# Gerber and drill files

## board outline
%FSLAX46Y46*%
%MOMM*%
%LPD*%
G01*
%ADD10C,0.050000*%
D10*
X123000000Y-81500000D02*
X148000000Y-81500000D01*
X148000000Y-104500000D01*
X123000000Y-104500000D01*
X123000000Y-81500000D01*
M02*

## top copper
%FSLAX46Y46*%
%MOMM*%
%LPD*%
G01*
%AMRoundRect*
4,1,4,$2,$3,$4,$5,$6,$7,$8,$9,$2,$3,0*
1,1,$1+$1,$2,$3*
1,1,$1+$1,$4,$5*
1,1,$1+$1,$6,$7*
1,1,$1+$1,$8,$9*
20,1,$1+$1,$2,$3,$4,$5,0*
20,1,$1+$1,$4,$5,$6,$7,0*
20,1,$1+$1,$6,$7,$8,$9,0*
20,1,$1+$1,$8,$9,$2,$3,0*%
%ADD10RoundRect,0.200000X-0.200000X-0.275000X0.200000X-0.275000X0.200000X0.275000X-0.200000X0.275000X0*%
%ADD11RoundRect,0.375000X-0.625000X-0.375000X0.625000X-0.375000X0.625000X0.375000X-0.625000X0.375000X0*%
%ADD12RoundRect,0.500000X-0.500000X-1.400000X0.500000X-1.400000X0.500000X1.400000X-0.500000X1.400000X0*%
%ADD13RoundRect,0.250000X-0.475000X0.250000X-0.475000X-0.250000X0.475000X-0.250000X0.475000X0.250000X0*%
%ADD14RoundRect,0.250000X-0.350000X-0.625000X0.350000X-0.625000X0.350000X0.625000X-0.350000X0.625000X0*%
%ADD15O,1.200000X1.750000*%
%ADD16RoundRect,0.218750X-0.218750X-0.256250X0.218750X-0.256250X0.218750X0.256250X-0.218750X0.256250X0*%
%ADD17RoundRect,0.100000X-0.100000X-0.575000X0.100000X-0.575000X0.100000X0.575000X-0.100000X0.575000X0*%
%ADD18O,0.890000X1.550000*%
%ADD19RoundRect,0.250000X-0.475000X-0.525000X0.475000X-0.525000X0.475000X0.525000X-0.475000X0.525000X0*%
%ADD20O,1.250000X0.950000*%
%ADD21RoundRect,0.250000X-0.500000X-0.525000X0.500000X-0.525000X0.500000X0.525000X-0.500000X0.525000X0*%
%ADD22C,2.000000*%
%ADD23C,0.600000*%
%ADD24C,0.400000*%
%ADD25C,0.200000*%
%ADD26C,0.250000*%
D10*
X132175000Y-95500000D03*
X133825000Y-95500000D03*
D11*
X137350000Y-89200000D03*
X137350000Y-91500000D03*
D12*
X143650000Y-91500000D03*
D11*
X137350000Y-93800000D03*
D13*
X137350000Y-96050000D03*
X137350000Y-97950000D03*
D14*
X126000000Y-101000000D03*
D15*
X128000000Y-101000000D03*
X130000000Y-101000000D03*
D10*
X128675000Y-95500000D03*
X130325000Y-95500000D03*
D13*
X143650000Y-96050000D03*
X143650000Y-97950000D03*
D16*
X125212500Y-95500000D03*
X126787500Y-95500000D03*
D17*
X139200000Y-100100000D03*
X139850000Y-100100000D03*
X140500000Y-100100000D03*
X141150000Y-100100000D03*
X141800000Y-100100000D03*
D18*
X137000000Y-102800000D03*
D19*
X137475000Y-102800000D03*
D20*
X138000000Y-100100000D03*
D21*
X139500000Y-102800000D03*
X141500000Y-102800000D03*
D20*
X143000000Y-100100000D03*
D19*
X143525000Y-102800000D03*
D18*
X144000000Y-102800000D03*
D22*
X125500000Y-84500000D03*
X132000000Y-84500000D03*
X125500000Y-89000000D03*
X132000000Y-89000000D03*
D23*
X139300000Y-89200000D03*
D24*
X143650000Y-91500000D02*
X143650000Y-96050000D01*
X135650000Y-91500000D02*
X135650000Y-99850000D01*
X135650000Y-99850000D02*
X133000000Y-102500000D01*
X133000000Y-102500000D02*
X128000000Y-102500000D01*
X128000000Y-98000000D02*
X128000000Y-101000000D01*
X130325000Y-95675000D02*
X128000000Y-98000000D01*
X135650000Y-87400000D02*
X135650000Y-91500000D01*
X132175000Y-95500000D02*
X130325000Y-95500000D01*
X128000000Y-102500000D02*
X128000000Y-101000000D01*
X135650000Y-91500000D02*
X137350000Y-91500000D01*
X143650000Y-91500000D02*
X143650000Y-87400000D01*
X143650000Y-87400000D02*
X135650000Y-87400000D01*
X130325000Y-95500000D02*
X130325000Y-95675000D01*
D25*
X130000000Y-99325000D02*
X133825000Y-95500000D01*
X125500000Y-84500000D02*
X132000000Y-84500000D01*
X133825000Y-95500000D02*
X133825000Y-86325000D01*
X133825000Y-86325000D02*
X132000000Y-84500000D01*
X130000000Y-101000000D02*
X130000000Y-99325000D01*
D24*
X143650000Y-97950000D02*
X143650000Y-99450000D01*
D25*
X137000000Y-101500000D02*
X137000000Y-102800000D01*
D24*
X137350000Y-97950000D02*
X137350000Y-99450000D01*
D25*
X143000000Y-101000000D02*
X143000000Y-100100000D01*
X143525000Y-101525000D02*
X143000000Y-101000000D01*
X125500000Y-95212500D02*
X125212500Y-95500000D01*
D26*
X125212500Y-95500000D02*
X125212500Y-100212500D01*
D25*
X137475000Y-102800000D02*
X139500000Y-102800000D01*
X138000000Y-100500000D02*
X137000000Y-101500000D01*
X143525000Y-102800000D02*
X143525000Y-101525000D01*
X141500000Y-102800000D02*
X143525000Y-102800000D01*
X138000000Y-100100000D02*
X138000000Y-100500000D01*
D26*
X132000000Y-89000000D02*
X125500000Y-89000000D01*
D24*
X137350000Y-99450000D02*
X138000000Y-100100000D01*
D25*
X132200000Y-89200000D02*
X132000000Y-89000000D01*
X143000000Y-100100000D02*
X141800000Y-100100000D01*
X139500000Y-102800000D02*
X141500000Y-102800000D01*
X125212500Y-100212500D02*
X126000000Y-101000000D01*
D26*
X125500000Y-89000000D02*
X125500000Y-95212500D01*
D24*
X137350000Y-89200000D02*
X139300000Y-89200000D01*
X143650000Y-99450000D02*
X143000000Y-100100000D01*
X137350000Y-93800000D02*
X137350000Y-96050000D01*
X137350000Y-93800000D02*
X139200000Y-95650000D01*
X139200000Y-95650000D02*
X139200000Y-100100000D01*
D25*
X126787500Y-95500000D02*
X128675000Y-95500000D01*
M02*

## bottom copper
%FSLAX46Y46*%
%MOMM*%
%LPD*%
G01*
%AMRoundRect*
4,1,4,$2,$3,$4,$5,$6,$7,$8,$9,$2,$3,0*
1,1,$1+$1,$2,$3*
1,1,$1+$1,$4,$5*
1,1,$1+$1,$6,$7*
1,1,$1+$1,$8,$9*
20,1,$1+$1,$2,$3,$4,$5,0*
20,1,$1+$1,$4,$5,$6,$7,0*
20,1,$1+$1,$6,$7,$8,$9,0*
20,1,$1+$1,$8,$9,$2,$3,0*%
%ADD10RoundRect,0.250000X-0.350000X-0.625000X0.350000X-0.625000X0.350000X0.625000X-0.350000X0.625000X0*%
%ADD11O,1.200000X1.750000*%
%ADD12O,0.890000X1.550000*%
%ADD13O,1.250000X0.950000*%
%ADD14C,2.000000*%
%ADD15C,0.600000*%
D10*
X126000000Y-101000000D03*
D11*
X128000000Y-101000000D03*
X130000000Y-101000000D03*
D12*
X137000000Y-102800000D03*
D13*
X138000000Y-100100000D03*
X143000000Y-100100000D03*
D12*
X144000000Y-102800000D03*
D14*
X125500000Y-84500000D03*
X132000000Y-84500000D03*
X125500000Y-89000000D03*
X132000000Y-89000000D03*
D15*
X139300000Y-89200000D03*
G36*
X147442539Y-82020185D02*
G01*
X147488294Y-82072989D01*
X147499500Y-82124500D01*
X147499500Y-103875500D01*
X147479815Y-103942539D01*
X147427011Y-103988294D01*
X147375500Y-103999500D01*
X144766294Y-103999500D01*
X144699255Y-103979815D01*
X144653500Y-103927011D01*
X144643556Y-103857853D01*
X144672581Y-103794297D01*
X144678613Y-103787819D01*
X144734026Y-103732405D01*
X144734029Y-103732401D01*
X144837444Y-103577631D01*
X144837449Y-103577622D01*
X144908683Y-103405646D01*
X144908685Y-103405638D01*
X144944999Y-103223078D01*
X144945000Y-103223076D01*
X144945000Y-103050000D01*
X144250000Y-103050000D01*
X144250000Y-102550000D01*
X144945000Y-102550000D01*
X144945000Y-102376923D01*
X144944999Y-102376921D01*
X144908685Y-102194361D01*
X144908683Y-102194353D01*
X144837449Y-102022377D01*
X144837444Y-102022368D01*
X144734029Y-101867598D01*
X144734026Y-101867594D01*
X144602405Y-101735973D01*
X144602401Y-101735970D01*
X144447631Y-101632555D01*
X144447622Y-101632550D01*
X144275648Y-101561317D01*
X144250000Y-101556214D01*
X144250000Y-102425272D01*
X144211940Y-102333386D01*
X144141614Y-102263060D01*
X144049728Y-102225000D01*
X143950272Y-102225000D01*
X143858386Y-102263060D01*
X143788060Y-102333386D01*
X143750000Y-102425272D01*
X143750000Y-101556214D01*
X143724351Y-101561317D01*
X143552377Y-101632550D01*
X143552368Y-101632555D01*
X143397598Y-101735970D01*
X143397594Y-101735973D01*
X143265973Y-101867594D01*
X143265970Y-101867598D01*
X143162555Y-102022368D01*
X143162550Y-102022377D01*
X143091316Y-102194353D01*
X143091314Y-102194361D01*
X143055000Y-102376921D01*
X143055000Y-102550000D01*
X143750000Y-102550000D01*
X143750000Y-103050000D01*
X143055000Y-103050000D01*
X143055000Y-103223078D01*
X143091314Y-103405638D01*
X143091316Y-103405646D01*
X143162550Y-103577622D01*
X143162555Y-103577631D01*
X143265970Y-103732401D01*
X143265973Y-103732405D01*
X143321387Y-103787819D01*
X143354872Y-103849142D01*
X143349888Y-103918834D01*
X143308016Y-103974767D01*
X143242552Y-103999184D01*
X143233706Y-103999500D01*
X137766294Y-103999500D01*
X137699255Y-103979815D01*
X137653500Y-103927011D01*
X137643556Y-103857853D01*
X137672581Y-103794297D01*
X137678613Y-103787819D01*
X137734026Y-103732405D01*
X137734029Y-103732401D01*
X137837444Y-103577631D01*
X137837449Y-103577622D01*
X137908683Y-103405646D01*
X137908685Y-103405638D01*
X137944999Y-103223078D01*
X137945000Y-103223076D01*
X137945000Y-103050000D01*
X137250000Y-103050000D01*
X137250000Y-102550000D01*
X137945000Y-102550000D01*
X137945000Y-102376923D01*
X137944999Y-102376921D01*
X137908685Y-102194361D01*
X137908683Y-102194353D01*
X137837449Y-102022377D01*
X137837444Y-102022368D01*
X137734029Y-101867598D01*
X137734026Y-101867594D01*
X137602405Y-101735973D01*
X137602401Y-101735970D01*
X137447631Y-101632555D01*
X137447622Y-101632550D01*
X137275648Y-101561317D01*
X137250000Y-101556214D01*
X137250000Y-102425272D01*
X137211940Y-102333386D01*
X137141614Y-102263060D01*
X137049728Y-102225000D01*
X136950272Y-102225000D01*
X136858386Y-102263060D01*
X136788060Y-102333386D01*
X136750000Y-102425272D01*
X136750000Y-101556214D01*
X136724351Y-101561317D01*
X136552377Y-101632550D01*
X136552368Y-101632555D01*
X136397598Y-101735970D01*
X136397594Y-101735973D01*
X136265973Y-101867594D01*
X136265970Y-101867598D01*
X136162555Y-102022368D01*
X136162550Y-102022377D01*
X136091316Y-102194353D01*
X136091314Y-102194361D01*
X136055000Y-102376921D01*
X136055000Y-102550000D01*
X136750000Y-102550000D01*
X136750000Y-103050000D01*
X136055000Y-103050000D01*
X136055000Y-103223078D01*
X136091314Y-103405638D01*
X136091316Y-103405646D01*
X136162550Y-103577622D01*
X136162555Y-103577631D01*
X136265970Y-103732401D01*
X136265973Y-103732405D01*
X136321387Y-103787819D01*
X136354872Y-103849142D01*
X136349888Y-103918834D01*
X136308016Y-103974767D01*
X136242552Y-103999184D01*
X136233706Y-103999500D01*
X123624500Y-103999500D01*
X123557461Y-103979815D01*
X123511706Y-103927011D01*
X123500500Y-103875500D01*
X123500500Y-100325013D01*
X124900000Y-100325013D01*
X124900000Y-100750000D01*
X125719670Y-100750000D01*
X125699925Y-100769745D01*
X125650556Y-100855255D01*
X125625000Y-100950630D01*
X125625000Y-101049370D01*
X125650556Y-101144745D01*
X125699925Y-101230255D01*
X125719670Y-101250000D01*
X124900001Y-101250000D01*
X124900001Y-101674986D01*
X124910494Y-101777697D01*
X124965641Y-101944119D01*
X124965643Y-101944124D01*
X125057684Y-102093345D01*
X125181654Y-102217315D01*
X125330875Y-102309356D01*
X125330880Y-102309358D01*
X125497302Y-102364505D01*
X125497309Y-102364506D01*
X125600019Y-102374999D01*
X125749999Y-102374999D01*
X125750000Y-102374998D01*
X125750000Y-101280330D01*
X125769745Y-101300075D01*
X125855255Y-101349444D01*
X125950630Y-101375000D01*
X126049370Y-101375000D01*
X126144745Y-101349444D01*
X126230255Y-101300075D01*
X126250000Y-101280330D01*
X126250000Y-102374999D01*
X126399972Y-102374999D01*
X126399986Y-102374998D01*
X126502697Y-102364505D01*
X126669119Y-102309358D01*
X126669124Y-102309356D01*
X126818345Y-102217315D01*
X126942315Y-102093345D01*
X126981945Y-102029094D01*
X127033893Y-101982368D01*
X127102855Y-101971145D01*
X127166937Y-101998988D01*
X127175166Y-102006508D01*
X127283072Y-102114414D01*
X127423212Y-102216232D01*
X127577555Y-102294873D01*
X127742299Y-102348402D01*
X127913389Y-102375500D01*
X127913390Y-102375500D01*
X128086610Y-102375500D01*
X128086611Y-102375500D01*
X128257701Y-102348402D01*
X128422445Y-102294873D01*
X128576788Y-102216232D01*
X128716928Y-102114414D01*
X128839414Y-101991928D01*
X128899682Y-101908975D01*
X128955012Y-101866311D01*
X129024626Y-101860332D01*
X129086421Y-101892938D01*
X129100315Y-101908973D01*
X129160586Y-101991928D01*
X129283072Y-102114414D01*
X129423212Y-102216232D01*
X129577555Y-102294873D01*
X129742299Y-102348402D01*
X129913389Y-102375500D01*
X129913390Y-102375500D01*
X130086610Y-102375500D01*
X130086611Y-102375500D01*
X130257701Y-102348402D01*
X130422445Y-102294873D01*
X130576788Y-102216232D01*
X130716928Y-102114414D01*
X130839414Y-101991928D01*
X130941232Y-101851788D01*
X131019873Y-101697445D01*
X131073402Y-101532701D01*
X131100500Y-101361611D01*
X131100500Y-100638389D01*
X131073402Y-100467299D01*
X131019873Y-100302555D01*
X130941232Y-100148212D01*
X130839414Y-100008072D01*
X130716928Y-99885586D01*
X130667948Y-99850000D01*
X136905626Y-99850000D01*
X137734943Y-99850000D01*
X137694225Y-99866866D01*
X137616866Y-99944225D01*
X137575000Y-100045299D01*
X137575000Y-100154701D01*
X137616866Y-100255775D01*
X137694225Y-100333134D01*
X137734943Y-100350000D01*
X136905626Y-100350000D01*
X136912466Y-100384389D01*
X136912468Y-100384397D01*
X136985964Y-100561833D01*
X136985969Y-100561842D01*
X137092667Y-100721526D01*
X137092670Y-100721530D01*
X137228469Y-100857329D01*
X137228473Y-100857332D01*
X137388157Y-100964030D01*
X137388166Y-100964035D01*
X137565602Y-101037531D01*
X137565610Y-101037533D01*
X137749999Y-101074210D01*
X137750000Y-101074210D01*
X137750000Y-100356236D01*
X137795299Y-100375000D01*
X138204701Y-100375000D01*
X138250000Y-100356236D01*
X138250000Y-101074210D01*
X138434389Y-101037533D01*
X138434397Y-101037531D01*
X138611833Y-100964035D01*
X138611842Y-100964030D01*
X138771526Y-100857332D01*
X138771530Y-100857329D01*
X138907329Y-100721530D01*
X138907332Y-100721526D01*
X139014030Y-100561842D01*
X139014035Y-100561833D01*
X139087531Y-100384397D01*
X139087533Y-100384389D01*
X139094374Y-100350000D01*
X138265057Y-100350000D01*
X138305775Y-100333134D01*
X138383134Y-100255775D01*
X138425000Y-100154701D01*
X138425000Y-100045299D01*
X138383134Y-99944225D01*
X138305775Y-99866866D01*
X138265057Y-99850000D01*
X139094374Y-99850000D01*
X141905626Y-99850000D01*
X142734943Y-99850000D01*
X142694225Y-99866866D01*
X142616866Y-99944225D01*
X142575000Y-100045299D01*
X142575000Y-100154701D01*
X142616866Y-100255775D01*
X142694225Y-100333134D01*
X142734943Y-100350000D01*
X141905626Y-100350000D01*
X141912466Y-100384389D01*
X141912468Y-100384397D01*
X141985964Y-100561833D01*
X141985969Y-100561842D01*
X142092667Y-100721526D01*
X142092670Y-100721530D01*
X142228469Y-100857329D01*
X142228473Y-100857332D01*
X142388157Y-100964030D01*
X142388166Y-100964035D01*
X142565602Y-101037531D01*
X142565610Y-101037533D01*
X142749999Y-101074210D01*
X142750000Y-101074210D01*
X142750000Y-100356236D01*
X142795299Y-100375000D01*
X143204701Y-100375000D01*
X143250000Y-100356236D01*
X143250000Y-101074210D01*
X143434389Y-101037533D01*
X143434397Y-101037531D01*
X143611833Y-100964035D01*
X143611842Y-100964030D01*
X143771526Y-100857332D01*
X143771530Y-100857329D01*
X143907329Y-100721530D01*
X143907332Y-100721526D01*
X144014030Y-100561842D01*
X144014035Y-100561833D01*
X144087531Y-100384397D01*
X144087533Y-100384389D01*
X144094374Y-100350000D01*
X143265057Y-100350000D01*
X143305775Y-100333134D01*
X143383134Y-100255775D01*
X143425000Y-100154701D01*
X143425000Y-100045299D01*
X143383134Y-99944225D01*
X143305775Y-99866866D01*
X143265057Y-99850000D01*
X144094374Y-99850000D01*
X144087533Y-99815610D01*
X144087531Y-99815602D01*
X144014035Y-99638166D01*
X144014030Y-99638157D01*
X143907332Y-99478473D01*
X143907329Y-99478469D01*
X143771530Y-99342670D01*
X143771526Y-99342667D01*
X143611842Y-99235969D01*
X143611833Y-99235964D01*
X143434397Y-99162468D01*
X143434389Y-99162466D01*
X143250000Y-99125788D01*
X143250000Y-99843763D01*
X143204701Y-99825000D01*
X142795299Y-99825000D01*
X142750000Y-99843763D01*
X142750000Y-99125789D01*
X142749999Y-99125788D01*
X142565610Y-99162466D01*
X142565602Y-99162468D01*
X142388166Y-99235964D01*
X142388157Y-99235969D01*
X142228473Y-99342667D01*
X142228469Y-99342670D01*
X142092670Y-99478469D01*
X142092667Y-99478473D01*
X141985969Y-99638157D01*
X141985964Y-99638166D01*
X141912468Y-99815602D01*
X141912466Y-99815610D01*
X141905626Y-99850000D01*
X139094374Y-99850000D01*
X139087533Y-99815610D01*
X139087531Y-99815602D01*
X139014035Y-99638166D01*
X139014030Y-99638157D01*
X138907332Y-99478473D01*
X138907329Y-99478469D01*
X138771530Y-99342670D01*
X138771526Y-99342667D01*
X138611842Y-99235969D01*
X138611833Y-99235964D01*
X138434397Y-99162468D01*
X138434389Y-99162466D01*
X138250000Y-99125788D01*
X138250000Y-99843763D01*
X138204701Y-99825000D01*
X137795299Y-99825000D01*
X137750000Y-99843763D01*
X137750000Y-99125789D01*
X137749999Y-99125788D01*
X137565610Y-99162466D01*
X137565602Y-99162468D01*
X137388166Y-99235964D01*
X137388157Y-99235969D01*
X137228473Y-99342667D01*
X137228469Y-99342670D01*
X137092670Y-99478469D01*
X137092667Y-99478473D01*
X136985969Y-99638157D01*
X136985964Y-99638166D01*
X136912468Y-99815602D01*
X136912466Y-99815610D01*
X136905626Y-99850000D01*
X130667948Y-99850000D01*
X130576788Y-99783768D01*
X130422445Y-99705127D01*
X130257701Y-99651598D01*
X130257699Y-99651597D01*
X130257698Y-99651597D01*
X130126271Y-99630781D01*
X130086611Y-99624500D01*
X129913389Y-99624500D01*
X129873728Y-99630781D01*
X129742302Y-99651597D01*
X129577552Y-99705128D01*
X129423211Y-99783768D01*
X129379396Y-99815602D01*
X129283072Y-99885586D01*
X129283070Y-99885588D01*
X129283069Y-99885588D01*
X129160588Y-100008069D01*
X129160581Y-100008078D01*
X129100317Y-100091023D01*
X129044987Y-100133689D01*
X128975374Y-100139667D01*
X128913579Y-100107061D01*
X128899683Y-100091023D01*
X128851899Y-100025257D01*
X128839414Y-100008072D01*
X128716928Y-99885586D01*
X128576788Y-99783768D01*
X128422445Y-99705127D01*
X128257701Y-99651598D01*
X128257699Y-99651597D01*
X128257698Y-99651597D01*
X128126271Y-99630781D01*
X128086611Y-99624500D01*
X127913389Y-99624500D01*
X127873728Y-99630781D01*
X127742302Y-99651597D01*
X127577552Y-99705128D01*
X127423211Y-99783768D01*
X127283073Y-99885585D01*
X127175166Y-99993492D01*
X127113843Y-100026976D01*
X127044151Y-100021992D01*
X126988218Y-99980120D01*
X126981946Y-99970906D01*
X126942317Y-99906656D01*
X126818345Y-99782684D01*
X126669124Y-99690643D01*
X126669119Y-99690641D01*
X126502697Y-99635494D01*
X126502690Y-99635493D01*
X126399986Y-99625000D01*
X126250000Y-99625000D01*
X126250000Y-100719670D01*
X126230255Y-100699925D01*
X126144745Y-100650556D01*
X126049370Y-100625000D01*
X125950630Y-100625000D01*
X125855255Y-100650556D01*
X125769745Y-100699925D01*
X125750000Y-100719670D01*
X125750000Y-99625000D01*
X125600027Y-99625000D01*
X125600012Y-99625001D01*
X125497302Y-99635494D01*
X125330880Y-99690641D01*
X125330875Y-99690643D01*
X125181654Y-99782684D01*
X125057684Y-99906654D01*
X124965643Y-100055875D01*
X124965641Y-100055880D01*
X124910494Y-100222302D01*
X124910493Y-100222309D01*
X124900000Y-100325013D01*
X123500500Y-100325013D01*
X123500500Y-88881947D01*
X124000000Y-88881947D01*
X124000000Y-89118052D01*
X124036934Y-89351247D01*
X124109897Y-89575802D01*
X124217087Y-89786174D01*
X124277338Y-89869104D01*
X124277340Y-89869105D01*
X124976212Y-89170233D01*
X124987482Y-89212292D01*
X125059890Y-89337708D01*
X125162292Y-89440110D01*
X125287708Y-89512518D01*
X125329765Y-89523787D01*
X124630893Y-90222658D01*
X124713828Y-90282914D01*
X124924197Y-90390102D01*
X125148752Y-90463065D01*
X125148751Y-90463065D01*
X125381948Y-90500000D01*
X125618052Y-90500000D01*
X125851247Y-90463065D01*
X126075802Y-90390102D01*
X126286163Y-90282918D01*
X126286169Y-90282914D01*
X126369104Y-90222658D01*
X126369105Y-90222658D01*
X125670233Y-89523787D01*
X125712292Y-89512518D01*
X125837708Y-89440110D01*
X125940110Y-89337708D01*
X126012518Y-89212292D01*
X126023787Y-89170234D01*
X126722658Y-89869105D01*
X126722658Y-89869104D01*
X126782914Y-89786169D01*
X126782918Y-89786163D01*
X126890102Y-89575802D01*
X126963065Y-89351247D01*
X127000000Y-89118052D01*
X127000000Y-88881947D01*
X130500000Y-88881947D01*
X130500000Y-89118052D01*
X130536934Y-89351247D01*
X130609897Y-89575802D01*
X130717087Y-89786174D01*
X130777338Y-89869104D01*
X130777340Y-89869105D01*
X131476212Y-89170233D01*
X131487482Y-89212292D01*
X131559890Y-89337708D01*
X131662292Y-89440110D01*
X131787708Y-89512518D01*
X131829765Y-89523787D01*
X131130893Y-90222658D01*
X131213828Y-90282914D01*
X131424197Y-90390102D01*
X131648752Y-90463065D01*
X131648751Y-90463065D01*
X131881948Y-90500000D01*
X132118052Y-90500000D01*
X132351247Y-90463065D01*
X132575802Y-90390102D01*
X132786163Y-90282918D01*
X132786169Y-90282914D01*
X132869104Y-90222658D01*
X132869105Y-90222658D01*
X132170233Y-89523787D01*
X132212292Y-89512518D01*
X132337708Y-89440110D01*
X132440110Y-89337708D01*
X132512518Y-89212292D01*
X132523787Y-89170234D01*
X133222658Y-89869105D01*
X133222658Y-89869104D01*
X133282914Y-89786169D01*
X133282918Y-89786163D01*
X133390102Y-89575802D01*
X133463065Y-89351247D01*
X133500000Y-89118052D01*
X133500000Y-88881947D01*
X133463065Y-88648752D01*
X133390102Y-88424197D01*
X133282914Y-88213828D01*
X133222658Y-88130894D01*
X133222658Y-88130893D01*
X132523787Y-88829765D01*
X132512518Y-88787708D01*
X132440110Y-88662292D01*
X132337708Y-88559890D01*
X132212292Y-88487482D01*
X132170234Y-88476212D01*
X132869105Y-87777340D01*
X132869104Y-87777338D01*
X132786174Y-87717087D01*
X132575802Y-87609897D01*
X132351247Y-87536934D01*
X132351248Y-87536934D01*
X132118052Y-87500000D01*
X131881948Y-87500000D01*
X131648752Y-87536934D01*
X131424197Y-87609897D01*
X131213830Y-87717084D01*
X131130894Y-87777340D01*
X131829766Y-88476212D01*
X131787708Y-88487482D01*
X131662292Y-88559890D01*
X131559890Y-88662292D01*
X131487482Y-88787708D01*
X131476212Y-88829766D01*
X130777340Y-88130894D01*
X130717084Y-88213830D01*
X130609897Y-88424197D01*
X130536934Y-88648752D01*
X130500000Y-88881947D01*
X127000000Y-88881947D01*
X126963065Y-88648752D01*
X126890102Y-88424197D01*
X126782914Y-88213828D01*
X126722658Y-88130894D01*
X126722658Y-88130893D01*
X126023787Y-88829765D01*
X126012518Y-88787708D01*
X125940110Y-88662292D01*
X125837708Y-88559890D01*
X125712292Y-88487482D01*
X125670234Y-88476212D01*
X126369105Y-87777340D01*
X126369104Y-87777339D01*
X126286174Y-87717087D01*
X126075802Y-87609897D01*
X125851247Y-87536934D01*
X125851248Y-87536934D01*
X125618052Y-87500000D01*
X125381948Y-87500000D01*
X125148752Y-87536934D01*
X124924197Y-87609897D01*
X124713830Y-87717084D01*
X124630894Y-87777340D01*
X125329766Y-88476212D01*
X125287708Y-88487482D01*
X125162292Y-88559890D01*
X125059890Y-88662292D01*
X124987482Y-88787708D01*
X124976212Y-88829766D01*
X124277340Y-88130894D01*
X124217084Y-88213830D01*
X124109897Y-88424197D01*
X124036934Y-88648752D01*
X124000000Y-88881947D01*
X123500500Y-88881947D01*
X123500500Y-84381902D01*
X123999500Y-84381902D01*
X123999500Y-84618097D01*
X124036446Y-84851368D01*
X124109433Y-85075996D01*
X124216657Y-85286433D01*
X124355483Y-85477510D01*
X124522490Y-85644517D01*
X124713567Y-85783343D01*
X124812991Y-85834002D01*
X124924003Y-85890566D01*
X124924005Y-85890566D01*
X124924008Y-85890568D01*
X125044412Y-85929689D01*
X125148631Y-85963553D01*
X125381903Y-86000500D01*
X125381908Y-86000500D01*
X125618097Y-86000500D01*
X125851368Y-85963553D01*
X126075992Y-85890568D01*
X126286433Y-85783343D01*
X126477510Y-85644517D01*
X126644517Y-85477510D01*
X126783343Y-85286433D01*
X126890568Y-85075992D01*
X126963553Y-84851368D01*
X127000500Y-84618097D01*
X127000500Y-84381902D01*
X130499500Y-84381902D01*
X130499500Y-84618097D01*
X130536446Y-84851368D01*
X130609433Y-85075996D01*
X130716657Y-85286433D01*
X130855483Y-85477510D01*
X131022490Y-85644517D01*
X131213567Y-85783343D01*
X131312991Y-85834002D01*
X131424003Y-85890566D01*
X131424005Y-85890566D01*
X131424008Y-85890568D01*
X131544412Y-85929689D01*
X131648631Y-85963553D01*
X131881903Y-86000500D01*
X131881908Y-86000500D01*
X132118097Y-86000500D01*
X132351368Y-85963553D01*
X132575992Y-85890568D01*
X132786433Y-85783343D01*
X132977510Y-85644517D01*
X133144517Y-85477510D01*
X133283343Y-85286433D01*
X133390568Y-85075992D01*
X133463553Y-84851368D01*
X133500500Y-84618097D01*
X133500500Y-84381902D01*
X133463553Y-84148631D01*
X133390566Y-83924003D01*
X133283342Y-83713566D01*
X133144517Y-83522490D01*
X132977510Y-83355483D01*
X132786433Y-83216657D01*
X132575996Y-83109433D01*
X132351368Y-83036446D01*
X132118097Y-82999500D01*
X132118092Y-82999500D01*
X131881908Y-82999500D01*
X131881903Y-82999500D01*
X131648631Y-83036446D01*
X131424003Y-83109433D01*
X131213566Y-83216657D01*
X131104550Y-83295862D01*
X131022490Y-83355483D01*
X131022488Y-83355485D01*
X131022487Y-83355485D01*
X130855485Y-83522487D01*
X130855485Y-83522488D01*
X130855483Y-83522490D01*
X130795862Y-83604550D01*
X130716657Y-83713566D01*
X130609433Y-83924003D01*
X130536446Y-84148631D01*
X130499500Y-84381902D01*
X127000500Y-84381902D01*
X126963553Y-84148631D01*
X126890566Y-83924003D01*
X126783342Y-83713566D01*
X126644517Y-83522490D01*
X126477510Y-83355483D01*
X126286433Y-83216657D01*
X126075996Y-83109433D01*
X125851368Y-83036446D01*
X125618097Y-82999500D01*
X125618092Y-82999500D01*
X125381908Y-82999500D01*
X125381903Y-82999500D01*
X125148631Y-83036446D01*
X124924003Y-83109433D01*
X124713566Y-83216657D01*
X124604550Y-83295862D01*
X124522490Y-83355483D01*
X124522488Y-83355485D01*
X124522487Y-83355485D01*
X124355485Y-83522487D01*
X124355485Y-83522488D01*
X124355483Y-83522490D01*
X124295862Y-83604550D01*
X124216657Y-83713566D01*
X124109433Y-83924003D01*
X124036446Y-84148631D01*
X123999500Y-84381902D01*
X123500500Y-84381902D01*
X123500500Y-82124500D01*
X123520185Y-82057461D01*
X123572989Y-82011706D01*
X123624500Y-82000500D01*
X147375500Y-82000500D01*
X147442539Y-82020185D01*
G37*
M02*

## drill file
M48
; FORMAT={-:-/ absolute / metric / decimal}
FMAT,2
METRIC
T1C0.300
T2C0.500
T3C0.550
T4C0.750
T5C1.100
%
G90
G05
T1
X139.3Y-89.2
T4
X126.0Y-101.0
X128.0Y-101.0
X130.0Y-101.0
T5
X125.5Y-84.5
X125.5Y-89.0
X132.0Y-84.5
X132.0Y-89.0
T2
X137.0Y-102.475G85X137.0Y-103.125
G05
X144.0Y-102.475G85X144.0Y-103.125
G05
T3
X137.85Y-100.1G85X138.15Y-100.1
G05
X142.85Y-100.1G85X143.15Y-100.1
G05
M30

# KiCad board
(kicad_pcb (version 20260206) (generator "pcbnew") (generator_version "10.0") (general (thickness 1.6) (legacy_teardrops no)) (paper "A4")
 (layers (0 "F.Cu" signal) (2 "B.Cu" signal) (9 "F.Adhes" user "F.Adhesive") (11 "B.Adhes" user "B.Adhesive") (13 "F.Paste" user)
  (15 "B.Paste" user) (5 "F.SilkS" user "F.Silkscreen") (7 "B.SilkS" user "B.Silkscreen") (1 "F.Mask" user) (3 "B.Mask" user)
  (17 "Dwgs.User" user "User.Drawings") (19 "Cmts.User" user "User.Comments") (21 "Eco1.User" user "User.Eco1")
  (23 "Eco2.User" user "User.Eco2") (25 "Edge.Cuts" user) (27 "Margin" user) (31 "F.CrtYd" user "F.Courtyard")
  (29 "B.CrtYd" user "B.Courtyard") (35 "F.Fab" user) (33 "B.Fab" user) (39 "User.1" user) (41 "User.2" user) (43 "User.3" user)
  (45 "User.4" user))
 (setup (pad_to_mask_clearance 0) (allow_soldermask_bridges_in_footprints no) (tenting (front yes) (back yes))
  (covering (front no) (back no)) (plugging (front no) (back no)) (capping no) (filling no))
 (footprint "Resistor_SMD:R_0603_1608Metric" (layer "F.Cu") (at 133 95.5)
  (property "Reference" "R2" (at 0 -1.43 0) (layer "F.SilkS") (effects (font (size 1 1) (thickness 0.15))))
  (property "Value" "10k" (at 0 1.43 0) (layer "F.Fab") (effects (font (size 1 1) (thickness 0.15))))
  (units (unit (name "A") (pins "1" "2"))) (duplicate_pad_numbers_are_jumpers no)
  (pad "1" smd roundrect (at -0.825 0) (size 0.8 0.95) (layers "F.Cu" "F.Mask" "F.Paste") (roundrect_rratio 0.25) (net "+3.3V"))
  (pad "2" smd roundrect (at 0.825 0) (size 0.8 0.95) (layers "F.Cu" "F.Mask" "F.Paste") (roundrect_rratio 0.25) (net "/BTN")))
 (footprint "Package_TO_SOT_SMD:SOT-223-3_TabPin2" (layer "F.Cu") (at 140.5 91.5)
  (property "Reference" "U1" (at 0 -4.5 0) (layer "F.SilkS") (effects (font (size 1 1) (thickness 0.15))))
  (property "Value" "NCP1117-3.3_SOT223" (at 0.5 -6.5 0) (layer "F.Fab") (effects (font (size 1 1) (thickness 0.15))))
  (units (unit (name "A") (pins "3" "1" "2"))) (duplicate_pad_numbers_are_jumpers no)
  (pad "1" smd roundrect (at -3.15 -2.3) (size 2 1.5) (layers "F.Cu" "F.Mask" "F.Paste") (roundrect_rratio 0.25) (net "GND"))
  (pad "2" smd roundrect (at -3.15 0) (size 2 1.5) (layers "F.Cu" "F.Mask" "F.Paste") (roundrect_rratio 0.25) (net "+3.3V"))
  (pad "2" smd roundrect (at 3.15 0) (size 2 3.8) (layers "F.Cu" "F.Mask" "F.Paste") (roundrect_rratio 0.25) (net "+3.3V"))
  (pad "3" smd roundrect (at -3.15 2.3) (size 2 1.5) (layers "F.Cu" "F.Mask" "F.Paste") (roundrect_rratio 0.25) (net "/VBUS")))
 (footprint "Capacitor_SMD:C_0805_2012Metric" (layer "F.Cu") (at 137.35 97 -90)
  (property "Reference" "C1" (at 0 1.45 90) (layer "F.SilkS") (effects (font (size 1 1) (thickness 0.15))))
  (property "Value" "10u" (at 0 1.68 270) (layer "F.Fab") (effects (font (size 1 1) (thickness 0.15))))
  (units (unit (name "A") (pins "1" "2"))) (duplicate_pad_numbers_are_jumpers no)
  (pad "1" smd roundrect (at -0.95 0 270) (size 1 1.45) (layers "F.Cu" "F.Mask" "F.Paste") (roundrect_rratio 0.25) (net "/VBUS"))
  (pad "2" smd roundrect (at 0.95 0 270) (size 1 1.45) (layers "F.Cu" "F.Mask" "F.Paste") (roundrect_rratio 0.25) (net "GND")))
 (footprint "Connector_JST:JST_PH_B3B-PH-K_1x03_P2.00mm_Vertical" (layer "F.Cu") (at 126 101)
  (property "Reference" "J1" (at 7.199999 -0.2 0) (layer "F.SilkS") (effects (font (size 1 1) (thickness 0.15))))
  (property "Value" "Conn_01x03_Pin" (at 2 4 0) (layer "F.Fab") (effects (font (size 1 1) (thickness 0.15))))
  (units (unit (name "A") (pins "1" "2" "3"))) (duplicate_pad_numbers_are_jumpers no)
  (pad "1" thru_hole roundrect (at 0 0) (size 1.2 1.75) (drill 0.75) (layers "*.Cu" "*.Mask") (remove_unused_layers no)
   (roundrect_rratio 0.208333) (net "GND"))
  (pad "2" thru_hole oval (at 2 0) (size 1.2 1.75) (drill 0.75) (layers "*.Cu" "*.Mask") (remove_unused_layers no) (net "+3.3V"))
  (pad "3" thru_hole oval (at 4 0) (size 1.2 1.75) (drill 0.75) (layers "*.Cu" "*.Mask") (remove_unused_layers no) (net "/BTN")))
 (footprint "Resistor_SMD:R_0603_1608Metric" (layer "F.Cu") (at 129.5 95.5)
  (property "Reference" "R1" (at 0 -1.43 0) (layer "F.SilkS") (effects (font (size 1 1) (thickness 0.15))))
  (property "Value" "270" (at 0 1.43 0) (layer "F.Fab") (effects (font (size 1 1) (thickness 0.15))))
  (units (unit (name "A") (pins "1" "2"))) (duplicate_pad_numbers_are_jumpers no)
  (pad "1" smd roundrect (at -0.825 0) (size 0.8 0.95) (layers "F.Cu" "F.Mask" "F.Paste") (roundrect_rratio 0.25) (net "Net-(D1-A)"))
  (pad "2" smd roundrect (at 0.825 0) (size 0.8 0.95) (layers "F.Cu" "F.Mask" "F.Paste") (roundrect_rratio 0.25) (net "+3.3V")))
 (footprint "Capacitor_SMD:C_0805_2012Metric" (layer "F.Cu") (at 143.65 97 -90)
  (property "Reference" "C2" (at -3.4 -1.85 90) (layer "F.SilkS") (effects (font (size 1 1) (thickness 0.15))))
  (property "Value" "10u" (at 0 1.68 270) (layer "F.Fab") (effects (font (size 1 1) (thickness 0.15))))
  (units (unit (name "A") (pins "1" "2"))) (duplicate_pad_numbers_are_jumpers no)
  (pad "1" smd roundrect (at -0.95 0 270) (size 1 1.45) (layers "F.Cu" "F.Mask" "F.Paste") (roundrect_rratio 0.25) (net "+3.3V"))
  (pad "2" smd roundrect (at 0.95 0 270) (size 1 1.45) (layers "F.Cu" "F.Mask" "F.Paste") (roundrect_rratio 0.25) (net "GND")))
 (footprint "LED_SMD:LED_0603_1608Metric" (layer "F.Cu") (at 126 95.5)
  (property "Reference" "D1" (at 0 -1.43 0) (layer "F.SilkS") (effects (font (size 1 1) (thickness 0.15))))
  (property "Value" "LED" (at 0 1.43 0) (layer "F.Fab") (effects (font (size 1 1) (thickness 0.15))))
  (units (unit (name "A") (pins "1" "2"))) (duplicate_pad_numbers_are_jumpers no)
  (pad "1" smd roundrect (at -0.7875 0) (size 0.875 0.95) (layers "F.Cu" "F.Mask" "F.Paste") (roundrect_rratio 0.25) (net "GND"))
  (pad "2" smd roundrect (at 0.7875 0) (size 0.875 0.95) (layers "F.Cu" "F.Mask" "F.Paste") (roundrect_rratio 0.25) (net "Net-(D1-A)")))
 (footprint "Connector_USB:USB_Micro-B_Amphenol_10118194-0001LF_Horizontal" (layer "F.Cu") (at 140.5 101.5)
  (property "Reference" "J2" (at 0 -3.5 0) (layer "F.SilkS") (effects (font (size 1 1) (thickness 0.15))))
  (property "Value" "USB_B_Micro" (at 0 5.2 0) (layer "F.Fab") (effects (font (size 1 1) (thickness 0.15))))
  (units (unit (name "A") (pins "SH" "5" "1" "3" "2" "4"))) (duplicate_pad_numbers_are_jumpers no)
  (pad "" smd oval (at -3.5 1.3) (size 0.89 1.55) (layers "F.Paste"))
  (pad "" smd oval (at -2.5 -1.4) (size 1.25 0.95) (layers "F.Paste"))
  (pad "" smd oval (at 2.5 -1.4) (size 1.25 0.95) (layers "F.Paste"))
  (pad "" smd oval (at 3.5 1.3) (size 0.89 1.55) (layers "F.Paste"))
  (pad "1" smd roundrect (at -1.3 -1.4) (size 0.4 1.35) (layers "F.Cu" "F.Mask" "F.Paste") (roundrect_rratio 0.25) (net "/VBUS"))
  (pad "2" smd roundrect (at -0.65 -1.4) (size 0.4 1.35) (layers "F.Cu" "F.Mask" "F.Paste") (roundrect_rratio 0.25)
   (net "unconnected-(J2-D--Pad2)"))
  (pad "3" smd roundrect (at 0 -1.4) (size 0.4 1.35) (layers "F.Cu" "F.Mask" "F.Paste") (roundrect_rratio 0.25)
   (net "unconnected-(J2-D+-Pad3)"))
  (pad "4" smd roundrect (at 0.65 -1.4) (size 0.4 1.35) (layers "F.Cu" "F.Mask" "F.Paste") (roundrect_rratio 0.25)
   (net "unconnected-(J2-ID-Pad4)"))
  (pad "5" smd roundrect (at 1.3 -1.4) (size 0.4 1.35) (layers "F.Cu" "F.Mask" "F.Paste") (roundrect_rratio 0.25) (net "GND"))
  (pad "SH" thru_hole oval (at -3.5 1.3) (size 0.89 1.55) (drill oval 0.5 1.15) (layers "*.Cu" "*.Mask") (remove_unused_layers no)
   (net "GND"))
  (pad "SH" smd roundrect (at -3.025 1.3) (size 1.45 1.55) (layers "F.Cu" "F.Mask" "F.Paste") (roundrect_rratio 0.1724137931) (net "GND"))
  (pad "SH" thru_hole oval (at -2.5 -1.4) (size 1.25 0.95) (drill oval 0.85 0.55) (layers "*.Cu" "*.Mask") (remove_unused_layers no)
   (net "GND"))
  (pad "SH" smd roundrect (at -1 1.3) (size 1.5 1.55) (layers "F.Cu" "F.Mask" "F.Paste") (roundrect_rratio 0.1666666667) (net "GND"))
  (pad "SH" smd roundrect (at 1 1.3) (size 1.5 1.55) (layers "F.Cu" "F.Mask" "F.Paste") (roundrect_rratio 0.1666666667) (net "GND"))
  (pad "SH" thru_hole oval (at 2.5 -1.4) (size 1.25 0.95) (drill oval 0.85 0.55) (layers "*.Cu" "*.Mask") (remove_unused_layers no)
   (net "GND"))
  (pad "SH" smd roundrect (at 3.025 1.3) (size 1.45 1.55) (layers "F.Cu" "F.Mask" "F.Paste") (roundrect_rratio 0.1724137931) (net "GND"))
  (pad "SH" thru_hole oval (at 3.5 1.3) (size 0.89 1.55) (drill oval 0.5 1.15) (layers "*.Cu" "*.Mask") (remove_unused_layers no)
   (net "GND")))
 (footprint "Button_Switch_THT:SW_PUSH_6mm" (layer "F.Cu") (at 125.5 84.5)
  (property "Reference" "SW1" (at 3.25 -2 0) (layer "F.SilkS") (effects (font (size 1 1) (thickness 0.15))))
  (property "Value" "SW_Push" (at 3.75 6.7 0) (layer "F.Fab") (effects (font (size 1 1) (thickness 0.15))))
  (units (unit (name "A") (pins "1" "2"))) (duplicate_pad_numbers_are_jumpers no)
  (pad "1" thru_hole circle (at 0 0 90) (size 2 2) (drill 1.1) (layers "*.Cu" "*.Mask") (remove_unused_layers no) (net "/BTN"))
  (pad "1" thru_hole circle (at 6.5 0 90) (size 2 2) (drill 1.1) (layers "*.Cu" "*.Mask") (remove_unused_layers no) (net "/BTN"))
  (pad "2" thru_hole circle (at 0 4.5 90) (size 2 2) (drill 1.1) (layers "*.Cu" "*.Mask") (remove_unused_layers no) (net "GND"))
  (pad "2" thru_hole circle (at 6.5 4.5 90) (size 2 2) (drill 1.1) (layers "*.Cu" "*.Mask") (remove_unused_layers no) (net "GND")))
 (gr_rect (start 123 81.5) (end 148 104.5) (stroke (width 0.05) (type default)) (fill no) (layer "Edge.Cuts"))
 (segment (start 143.65 91.5) (end 143.65 96.05) (width 0.4) (layer "F.Cu") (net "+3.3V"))
 (segment (start 135.65 91.5) (end 135.65 99.85) (width 0.4) (layer "F.Cu") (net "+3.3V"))
 (segment (start 135.65 99.85) (end 133 102.5) (width 0.4) (layer "F.Cu") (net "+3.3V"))
 (segment (start 133 102.5) (end 128 102.5) (width 0.4) (layer "F.Cu") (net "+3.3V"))
 (segment (start 128 98) (end 128 101) (width 0.4) (layer "F.Cu") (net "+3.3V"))
 (segment (start 130.325 95.675) (end 128 98) (width 0.4) (layer "F.Cu") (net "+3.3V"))
 (segment (start 135.65 87.4) (end 135.65 91.5) (width 0.4) (layer "F.Cu") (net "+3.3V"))
 (segment (start 132.175 95.5) (end 130.325 95.5) (width 0.4) (layer "F.Cu") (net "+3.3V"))
 (segment (start 128 102.5) (end 128 101) (width 0.4) (layer "F.Cu") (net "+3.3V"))
 (segment (start 135.65 91.5) (end 137.35 91.5) (width 0.4) (layer "F.Cu") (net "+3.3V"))
 (segment (start 143.65 91.5) (end 143.65 87.4) (width 0.4) (layer "F.Cu") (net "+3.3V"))
 (segment (start 143.65 87.4) (end 135.65 87.4) (width 0.4) (layer "F.Cu") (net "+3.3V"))
 (segment (start 130.325 95.5) (end 130.325 95.675) (width 0.4) (layer "F.Cu") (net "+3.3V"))
 (segment (start 130 99.325) (end 133.825 95.5) (width 0.2) (layer "F.Cu") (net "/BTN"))
 (segment (start 125.5 84.5) (end 132 84.5) (width 0.2) (layer "F.Cu") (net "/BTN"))
 (segment (start 133.825 95.5) (end 133.825 86.325) (width 0.2) (layer "F.Cu") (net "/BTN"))
 (segment (start 133.825 86.325) (end 132 84.5) (width 0.2) (layer "F.Cu") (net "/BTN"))
 (segment (start 130 101) (end 130 99.325) (width 0.2) (layer "F.Cu") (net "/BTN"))
 (segment (start 143.65 97.95) (end 143.65 99.45) (width 0.4) (layer "F.Cu") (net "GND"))
 (segment (start 137 101.5) (end 137 102.8) (width 0.2) (layer "F.Cu") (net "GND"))
 (segment (start 137.35 97.95) (end 137.35 99.45) (width 0.4) (layer "F.Cu") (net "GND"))
 (segment (start 143 101) (end 143 100.1) (width 0.2) (layer "F.Cu") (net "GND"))
 (segment (start 143.525 101.525) (end 143 101) (width 0.2) (layer "F.Cu") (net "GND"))
 (segment (start 125.5 95.2125) (end 125.2125 95.5) (width 0.2) (layer "F.Cu") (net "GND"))
 (segment (start 125.2125 95.5) (end 125.2125 100.2125) (width 0.25) (layer "F.Cu") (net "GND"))
 (segment (start 137.475 102.8) (end 139.5 102.8) (width 0.2) (layer "F.Cu") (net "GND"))
 (segment (start 138 100.5) (end 137 101.5) (width 0.2) (layer "F.Cu") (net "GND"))
 (segment (start 143.525 102.8) (end 143.525 101.525) (width 0.2) (layer "F.Cu") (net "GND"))
 (segment (start 141.5 102.8) (end 143.525 102.8) (width 0.2) (layer "F.Cu") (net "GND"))
 (segment (start 138 100.1) (end 138 100.5) (width 0.2) (layer "F.Cu") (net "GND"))
 (segment (start 132 89) (end 125.5 89) (width 0.25) (layer "F.Cu") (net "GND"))
 (segment (start 137.35 99.45) (end 138 100.1) (width 0.4) (layer "F.Cu") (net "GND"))
 (segment (start 132.2 89.2) (end 132 89) (width 0.2) (layer "F.Cu") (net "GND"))
 (segment (start 143 100.1) (end 141.8 100.1) (width 0.2) (layer "F.Cu") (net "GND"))
 (segment (start 139.5 102.8) (end 141.5 102.8) (width 0.2) (layer "F.Cu") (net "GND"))
 (segment (start 125.2125 100.2125) (end 126 101) (width 0.2) (layer "F.Cu") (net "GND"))
 (segment (start 125.5 89) (end 125.5 95.2125) (width 0.25) (layer "F.Cu") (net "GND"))
 (segment (start 137.35 89.2) (end 139.3 89.2) (width 0.4) (layer "F.Cu") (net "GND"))
 (segment (start 143.65 99.45) (end 143 100.1) (width 0.4) (layer "F.Cu") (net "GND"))
 (via (at 139.3 89.2) (size 0.6) (drill 0.3) (layers "F.Cu" "B.Cu") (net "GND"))
 (segment (start 137.35 93.8) (end 137.35 96.05) (width 0.4) (layer "F.Cu") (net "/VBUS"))
 (segment (start 137.35 93.8) (end 139.2 95.65) (width 0.4) (layer "F.Cu") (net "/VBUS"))
 (segment (start 139.2 95.65) (end 139.2 100.1) (width 0.4) (layer "F.Cu") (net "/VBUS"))
 (segment (start 126.7875 95.5) (end 128.675 95.5) (width 0.2) (layer "F.Cu") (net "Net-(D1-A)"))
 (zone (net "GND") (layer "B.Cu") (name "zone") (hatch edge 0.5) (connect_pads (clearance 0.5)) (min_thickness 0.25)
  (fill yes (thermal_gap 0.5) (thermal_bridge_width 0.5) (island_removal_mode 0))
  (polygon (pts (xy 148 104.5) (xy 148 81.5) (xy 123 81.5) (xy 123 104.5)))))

